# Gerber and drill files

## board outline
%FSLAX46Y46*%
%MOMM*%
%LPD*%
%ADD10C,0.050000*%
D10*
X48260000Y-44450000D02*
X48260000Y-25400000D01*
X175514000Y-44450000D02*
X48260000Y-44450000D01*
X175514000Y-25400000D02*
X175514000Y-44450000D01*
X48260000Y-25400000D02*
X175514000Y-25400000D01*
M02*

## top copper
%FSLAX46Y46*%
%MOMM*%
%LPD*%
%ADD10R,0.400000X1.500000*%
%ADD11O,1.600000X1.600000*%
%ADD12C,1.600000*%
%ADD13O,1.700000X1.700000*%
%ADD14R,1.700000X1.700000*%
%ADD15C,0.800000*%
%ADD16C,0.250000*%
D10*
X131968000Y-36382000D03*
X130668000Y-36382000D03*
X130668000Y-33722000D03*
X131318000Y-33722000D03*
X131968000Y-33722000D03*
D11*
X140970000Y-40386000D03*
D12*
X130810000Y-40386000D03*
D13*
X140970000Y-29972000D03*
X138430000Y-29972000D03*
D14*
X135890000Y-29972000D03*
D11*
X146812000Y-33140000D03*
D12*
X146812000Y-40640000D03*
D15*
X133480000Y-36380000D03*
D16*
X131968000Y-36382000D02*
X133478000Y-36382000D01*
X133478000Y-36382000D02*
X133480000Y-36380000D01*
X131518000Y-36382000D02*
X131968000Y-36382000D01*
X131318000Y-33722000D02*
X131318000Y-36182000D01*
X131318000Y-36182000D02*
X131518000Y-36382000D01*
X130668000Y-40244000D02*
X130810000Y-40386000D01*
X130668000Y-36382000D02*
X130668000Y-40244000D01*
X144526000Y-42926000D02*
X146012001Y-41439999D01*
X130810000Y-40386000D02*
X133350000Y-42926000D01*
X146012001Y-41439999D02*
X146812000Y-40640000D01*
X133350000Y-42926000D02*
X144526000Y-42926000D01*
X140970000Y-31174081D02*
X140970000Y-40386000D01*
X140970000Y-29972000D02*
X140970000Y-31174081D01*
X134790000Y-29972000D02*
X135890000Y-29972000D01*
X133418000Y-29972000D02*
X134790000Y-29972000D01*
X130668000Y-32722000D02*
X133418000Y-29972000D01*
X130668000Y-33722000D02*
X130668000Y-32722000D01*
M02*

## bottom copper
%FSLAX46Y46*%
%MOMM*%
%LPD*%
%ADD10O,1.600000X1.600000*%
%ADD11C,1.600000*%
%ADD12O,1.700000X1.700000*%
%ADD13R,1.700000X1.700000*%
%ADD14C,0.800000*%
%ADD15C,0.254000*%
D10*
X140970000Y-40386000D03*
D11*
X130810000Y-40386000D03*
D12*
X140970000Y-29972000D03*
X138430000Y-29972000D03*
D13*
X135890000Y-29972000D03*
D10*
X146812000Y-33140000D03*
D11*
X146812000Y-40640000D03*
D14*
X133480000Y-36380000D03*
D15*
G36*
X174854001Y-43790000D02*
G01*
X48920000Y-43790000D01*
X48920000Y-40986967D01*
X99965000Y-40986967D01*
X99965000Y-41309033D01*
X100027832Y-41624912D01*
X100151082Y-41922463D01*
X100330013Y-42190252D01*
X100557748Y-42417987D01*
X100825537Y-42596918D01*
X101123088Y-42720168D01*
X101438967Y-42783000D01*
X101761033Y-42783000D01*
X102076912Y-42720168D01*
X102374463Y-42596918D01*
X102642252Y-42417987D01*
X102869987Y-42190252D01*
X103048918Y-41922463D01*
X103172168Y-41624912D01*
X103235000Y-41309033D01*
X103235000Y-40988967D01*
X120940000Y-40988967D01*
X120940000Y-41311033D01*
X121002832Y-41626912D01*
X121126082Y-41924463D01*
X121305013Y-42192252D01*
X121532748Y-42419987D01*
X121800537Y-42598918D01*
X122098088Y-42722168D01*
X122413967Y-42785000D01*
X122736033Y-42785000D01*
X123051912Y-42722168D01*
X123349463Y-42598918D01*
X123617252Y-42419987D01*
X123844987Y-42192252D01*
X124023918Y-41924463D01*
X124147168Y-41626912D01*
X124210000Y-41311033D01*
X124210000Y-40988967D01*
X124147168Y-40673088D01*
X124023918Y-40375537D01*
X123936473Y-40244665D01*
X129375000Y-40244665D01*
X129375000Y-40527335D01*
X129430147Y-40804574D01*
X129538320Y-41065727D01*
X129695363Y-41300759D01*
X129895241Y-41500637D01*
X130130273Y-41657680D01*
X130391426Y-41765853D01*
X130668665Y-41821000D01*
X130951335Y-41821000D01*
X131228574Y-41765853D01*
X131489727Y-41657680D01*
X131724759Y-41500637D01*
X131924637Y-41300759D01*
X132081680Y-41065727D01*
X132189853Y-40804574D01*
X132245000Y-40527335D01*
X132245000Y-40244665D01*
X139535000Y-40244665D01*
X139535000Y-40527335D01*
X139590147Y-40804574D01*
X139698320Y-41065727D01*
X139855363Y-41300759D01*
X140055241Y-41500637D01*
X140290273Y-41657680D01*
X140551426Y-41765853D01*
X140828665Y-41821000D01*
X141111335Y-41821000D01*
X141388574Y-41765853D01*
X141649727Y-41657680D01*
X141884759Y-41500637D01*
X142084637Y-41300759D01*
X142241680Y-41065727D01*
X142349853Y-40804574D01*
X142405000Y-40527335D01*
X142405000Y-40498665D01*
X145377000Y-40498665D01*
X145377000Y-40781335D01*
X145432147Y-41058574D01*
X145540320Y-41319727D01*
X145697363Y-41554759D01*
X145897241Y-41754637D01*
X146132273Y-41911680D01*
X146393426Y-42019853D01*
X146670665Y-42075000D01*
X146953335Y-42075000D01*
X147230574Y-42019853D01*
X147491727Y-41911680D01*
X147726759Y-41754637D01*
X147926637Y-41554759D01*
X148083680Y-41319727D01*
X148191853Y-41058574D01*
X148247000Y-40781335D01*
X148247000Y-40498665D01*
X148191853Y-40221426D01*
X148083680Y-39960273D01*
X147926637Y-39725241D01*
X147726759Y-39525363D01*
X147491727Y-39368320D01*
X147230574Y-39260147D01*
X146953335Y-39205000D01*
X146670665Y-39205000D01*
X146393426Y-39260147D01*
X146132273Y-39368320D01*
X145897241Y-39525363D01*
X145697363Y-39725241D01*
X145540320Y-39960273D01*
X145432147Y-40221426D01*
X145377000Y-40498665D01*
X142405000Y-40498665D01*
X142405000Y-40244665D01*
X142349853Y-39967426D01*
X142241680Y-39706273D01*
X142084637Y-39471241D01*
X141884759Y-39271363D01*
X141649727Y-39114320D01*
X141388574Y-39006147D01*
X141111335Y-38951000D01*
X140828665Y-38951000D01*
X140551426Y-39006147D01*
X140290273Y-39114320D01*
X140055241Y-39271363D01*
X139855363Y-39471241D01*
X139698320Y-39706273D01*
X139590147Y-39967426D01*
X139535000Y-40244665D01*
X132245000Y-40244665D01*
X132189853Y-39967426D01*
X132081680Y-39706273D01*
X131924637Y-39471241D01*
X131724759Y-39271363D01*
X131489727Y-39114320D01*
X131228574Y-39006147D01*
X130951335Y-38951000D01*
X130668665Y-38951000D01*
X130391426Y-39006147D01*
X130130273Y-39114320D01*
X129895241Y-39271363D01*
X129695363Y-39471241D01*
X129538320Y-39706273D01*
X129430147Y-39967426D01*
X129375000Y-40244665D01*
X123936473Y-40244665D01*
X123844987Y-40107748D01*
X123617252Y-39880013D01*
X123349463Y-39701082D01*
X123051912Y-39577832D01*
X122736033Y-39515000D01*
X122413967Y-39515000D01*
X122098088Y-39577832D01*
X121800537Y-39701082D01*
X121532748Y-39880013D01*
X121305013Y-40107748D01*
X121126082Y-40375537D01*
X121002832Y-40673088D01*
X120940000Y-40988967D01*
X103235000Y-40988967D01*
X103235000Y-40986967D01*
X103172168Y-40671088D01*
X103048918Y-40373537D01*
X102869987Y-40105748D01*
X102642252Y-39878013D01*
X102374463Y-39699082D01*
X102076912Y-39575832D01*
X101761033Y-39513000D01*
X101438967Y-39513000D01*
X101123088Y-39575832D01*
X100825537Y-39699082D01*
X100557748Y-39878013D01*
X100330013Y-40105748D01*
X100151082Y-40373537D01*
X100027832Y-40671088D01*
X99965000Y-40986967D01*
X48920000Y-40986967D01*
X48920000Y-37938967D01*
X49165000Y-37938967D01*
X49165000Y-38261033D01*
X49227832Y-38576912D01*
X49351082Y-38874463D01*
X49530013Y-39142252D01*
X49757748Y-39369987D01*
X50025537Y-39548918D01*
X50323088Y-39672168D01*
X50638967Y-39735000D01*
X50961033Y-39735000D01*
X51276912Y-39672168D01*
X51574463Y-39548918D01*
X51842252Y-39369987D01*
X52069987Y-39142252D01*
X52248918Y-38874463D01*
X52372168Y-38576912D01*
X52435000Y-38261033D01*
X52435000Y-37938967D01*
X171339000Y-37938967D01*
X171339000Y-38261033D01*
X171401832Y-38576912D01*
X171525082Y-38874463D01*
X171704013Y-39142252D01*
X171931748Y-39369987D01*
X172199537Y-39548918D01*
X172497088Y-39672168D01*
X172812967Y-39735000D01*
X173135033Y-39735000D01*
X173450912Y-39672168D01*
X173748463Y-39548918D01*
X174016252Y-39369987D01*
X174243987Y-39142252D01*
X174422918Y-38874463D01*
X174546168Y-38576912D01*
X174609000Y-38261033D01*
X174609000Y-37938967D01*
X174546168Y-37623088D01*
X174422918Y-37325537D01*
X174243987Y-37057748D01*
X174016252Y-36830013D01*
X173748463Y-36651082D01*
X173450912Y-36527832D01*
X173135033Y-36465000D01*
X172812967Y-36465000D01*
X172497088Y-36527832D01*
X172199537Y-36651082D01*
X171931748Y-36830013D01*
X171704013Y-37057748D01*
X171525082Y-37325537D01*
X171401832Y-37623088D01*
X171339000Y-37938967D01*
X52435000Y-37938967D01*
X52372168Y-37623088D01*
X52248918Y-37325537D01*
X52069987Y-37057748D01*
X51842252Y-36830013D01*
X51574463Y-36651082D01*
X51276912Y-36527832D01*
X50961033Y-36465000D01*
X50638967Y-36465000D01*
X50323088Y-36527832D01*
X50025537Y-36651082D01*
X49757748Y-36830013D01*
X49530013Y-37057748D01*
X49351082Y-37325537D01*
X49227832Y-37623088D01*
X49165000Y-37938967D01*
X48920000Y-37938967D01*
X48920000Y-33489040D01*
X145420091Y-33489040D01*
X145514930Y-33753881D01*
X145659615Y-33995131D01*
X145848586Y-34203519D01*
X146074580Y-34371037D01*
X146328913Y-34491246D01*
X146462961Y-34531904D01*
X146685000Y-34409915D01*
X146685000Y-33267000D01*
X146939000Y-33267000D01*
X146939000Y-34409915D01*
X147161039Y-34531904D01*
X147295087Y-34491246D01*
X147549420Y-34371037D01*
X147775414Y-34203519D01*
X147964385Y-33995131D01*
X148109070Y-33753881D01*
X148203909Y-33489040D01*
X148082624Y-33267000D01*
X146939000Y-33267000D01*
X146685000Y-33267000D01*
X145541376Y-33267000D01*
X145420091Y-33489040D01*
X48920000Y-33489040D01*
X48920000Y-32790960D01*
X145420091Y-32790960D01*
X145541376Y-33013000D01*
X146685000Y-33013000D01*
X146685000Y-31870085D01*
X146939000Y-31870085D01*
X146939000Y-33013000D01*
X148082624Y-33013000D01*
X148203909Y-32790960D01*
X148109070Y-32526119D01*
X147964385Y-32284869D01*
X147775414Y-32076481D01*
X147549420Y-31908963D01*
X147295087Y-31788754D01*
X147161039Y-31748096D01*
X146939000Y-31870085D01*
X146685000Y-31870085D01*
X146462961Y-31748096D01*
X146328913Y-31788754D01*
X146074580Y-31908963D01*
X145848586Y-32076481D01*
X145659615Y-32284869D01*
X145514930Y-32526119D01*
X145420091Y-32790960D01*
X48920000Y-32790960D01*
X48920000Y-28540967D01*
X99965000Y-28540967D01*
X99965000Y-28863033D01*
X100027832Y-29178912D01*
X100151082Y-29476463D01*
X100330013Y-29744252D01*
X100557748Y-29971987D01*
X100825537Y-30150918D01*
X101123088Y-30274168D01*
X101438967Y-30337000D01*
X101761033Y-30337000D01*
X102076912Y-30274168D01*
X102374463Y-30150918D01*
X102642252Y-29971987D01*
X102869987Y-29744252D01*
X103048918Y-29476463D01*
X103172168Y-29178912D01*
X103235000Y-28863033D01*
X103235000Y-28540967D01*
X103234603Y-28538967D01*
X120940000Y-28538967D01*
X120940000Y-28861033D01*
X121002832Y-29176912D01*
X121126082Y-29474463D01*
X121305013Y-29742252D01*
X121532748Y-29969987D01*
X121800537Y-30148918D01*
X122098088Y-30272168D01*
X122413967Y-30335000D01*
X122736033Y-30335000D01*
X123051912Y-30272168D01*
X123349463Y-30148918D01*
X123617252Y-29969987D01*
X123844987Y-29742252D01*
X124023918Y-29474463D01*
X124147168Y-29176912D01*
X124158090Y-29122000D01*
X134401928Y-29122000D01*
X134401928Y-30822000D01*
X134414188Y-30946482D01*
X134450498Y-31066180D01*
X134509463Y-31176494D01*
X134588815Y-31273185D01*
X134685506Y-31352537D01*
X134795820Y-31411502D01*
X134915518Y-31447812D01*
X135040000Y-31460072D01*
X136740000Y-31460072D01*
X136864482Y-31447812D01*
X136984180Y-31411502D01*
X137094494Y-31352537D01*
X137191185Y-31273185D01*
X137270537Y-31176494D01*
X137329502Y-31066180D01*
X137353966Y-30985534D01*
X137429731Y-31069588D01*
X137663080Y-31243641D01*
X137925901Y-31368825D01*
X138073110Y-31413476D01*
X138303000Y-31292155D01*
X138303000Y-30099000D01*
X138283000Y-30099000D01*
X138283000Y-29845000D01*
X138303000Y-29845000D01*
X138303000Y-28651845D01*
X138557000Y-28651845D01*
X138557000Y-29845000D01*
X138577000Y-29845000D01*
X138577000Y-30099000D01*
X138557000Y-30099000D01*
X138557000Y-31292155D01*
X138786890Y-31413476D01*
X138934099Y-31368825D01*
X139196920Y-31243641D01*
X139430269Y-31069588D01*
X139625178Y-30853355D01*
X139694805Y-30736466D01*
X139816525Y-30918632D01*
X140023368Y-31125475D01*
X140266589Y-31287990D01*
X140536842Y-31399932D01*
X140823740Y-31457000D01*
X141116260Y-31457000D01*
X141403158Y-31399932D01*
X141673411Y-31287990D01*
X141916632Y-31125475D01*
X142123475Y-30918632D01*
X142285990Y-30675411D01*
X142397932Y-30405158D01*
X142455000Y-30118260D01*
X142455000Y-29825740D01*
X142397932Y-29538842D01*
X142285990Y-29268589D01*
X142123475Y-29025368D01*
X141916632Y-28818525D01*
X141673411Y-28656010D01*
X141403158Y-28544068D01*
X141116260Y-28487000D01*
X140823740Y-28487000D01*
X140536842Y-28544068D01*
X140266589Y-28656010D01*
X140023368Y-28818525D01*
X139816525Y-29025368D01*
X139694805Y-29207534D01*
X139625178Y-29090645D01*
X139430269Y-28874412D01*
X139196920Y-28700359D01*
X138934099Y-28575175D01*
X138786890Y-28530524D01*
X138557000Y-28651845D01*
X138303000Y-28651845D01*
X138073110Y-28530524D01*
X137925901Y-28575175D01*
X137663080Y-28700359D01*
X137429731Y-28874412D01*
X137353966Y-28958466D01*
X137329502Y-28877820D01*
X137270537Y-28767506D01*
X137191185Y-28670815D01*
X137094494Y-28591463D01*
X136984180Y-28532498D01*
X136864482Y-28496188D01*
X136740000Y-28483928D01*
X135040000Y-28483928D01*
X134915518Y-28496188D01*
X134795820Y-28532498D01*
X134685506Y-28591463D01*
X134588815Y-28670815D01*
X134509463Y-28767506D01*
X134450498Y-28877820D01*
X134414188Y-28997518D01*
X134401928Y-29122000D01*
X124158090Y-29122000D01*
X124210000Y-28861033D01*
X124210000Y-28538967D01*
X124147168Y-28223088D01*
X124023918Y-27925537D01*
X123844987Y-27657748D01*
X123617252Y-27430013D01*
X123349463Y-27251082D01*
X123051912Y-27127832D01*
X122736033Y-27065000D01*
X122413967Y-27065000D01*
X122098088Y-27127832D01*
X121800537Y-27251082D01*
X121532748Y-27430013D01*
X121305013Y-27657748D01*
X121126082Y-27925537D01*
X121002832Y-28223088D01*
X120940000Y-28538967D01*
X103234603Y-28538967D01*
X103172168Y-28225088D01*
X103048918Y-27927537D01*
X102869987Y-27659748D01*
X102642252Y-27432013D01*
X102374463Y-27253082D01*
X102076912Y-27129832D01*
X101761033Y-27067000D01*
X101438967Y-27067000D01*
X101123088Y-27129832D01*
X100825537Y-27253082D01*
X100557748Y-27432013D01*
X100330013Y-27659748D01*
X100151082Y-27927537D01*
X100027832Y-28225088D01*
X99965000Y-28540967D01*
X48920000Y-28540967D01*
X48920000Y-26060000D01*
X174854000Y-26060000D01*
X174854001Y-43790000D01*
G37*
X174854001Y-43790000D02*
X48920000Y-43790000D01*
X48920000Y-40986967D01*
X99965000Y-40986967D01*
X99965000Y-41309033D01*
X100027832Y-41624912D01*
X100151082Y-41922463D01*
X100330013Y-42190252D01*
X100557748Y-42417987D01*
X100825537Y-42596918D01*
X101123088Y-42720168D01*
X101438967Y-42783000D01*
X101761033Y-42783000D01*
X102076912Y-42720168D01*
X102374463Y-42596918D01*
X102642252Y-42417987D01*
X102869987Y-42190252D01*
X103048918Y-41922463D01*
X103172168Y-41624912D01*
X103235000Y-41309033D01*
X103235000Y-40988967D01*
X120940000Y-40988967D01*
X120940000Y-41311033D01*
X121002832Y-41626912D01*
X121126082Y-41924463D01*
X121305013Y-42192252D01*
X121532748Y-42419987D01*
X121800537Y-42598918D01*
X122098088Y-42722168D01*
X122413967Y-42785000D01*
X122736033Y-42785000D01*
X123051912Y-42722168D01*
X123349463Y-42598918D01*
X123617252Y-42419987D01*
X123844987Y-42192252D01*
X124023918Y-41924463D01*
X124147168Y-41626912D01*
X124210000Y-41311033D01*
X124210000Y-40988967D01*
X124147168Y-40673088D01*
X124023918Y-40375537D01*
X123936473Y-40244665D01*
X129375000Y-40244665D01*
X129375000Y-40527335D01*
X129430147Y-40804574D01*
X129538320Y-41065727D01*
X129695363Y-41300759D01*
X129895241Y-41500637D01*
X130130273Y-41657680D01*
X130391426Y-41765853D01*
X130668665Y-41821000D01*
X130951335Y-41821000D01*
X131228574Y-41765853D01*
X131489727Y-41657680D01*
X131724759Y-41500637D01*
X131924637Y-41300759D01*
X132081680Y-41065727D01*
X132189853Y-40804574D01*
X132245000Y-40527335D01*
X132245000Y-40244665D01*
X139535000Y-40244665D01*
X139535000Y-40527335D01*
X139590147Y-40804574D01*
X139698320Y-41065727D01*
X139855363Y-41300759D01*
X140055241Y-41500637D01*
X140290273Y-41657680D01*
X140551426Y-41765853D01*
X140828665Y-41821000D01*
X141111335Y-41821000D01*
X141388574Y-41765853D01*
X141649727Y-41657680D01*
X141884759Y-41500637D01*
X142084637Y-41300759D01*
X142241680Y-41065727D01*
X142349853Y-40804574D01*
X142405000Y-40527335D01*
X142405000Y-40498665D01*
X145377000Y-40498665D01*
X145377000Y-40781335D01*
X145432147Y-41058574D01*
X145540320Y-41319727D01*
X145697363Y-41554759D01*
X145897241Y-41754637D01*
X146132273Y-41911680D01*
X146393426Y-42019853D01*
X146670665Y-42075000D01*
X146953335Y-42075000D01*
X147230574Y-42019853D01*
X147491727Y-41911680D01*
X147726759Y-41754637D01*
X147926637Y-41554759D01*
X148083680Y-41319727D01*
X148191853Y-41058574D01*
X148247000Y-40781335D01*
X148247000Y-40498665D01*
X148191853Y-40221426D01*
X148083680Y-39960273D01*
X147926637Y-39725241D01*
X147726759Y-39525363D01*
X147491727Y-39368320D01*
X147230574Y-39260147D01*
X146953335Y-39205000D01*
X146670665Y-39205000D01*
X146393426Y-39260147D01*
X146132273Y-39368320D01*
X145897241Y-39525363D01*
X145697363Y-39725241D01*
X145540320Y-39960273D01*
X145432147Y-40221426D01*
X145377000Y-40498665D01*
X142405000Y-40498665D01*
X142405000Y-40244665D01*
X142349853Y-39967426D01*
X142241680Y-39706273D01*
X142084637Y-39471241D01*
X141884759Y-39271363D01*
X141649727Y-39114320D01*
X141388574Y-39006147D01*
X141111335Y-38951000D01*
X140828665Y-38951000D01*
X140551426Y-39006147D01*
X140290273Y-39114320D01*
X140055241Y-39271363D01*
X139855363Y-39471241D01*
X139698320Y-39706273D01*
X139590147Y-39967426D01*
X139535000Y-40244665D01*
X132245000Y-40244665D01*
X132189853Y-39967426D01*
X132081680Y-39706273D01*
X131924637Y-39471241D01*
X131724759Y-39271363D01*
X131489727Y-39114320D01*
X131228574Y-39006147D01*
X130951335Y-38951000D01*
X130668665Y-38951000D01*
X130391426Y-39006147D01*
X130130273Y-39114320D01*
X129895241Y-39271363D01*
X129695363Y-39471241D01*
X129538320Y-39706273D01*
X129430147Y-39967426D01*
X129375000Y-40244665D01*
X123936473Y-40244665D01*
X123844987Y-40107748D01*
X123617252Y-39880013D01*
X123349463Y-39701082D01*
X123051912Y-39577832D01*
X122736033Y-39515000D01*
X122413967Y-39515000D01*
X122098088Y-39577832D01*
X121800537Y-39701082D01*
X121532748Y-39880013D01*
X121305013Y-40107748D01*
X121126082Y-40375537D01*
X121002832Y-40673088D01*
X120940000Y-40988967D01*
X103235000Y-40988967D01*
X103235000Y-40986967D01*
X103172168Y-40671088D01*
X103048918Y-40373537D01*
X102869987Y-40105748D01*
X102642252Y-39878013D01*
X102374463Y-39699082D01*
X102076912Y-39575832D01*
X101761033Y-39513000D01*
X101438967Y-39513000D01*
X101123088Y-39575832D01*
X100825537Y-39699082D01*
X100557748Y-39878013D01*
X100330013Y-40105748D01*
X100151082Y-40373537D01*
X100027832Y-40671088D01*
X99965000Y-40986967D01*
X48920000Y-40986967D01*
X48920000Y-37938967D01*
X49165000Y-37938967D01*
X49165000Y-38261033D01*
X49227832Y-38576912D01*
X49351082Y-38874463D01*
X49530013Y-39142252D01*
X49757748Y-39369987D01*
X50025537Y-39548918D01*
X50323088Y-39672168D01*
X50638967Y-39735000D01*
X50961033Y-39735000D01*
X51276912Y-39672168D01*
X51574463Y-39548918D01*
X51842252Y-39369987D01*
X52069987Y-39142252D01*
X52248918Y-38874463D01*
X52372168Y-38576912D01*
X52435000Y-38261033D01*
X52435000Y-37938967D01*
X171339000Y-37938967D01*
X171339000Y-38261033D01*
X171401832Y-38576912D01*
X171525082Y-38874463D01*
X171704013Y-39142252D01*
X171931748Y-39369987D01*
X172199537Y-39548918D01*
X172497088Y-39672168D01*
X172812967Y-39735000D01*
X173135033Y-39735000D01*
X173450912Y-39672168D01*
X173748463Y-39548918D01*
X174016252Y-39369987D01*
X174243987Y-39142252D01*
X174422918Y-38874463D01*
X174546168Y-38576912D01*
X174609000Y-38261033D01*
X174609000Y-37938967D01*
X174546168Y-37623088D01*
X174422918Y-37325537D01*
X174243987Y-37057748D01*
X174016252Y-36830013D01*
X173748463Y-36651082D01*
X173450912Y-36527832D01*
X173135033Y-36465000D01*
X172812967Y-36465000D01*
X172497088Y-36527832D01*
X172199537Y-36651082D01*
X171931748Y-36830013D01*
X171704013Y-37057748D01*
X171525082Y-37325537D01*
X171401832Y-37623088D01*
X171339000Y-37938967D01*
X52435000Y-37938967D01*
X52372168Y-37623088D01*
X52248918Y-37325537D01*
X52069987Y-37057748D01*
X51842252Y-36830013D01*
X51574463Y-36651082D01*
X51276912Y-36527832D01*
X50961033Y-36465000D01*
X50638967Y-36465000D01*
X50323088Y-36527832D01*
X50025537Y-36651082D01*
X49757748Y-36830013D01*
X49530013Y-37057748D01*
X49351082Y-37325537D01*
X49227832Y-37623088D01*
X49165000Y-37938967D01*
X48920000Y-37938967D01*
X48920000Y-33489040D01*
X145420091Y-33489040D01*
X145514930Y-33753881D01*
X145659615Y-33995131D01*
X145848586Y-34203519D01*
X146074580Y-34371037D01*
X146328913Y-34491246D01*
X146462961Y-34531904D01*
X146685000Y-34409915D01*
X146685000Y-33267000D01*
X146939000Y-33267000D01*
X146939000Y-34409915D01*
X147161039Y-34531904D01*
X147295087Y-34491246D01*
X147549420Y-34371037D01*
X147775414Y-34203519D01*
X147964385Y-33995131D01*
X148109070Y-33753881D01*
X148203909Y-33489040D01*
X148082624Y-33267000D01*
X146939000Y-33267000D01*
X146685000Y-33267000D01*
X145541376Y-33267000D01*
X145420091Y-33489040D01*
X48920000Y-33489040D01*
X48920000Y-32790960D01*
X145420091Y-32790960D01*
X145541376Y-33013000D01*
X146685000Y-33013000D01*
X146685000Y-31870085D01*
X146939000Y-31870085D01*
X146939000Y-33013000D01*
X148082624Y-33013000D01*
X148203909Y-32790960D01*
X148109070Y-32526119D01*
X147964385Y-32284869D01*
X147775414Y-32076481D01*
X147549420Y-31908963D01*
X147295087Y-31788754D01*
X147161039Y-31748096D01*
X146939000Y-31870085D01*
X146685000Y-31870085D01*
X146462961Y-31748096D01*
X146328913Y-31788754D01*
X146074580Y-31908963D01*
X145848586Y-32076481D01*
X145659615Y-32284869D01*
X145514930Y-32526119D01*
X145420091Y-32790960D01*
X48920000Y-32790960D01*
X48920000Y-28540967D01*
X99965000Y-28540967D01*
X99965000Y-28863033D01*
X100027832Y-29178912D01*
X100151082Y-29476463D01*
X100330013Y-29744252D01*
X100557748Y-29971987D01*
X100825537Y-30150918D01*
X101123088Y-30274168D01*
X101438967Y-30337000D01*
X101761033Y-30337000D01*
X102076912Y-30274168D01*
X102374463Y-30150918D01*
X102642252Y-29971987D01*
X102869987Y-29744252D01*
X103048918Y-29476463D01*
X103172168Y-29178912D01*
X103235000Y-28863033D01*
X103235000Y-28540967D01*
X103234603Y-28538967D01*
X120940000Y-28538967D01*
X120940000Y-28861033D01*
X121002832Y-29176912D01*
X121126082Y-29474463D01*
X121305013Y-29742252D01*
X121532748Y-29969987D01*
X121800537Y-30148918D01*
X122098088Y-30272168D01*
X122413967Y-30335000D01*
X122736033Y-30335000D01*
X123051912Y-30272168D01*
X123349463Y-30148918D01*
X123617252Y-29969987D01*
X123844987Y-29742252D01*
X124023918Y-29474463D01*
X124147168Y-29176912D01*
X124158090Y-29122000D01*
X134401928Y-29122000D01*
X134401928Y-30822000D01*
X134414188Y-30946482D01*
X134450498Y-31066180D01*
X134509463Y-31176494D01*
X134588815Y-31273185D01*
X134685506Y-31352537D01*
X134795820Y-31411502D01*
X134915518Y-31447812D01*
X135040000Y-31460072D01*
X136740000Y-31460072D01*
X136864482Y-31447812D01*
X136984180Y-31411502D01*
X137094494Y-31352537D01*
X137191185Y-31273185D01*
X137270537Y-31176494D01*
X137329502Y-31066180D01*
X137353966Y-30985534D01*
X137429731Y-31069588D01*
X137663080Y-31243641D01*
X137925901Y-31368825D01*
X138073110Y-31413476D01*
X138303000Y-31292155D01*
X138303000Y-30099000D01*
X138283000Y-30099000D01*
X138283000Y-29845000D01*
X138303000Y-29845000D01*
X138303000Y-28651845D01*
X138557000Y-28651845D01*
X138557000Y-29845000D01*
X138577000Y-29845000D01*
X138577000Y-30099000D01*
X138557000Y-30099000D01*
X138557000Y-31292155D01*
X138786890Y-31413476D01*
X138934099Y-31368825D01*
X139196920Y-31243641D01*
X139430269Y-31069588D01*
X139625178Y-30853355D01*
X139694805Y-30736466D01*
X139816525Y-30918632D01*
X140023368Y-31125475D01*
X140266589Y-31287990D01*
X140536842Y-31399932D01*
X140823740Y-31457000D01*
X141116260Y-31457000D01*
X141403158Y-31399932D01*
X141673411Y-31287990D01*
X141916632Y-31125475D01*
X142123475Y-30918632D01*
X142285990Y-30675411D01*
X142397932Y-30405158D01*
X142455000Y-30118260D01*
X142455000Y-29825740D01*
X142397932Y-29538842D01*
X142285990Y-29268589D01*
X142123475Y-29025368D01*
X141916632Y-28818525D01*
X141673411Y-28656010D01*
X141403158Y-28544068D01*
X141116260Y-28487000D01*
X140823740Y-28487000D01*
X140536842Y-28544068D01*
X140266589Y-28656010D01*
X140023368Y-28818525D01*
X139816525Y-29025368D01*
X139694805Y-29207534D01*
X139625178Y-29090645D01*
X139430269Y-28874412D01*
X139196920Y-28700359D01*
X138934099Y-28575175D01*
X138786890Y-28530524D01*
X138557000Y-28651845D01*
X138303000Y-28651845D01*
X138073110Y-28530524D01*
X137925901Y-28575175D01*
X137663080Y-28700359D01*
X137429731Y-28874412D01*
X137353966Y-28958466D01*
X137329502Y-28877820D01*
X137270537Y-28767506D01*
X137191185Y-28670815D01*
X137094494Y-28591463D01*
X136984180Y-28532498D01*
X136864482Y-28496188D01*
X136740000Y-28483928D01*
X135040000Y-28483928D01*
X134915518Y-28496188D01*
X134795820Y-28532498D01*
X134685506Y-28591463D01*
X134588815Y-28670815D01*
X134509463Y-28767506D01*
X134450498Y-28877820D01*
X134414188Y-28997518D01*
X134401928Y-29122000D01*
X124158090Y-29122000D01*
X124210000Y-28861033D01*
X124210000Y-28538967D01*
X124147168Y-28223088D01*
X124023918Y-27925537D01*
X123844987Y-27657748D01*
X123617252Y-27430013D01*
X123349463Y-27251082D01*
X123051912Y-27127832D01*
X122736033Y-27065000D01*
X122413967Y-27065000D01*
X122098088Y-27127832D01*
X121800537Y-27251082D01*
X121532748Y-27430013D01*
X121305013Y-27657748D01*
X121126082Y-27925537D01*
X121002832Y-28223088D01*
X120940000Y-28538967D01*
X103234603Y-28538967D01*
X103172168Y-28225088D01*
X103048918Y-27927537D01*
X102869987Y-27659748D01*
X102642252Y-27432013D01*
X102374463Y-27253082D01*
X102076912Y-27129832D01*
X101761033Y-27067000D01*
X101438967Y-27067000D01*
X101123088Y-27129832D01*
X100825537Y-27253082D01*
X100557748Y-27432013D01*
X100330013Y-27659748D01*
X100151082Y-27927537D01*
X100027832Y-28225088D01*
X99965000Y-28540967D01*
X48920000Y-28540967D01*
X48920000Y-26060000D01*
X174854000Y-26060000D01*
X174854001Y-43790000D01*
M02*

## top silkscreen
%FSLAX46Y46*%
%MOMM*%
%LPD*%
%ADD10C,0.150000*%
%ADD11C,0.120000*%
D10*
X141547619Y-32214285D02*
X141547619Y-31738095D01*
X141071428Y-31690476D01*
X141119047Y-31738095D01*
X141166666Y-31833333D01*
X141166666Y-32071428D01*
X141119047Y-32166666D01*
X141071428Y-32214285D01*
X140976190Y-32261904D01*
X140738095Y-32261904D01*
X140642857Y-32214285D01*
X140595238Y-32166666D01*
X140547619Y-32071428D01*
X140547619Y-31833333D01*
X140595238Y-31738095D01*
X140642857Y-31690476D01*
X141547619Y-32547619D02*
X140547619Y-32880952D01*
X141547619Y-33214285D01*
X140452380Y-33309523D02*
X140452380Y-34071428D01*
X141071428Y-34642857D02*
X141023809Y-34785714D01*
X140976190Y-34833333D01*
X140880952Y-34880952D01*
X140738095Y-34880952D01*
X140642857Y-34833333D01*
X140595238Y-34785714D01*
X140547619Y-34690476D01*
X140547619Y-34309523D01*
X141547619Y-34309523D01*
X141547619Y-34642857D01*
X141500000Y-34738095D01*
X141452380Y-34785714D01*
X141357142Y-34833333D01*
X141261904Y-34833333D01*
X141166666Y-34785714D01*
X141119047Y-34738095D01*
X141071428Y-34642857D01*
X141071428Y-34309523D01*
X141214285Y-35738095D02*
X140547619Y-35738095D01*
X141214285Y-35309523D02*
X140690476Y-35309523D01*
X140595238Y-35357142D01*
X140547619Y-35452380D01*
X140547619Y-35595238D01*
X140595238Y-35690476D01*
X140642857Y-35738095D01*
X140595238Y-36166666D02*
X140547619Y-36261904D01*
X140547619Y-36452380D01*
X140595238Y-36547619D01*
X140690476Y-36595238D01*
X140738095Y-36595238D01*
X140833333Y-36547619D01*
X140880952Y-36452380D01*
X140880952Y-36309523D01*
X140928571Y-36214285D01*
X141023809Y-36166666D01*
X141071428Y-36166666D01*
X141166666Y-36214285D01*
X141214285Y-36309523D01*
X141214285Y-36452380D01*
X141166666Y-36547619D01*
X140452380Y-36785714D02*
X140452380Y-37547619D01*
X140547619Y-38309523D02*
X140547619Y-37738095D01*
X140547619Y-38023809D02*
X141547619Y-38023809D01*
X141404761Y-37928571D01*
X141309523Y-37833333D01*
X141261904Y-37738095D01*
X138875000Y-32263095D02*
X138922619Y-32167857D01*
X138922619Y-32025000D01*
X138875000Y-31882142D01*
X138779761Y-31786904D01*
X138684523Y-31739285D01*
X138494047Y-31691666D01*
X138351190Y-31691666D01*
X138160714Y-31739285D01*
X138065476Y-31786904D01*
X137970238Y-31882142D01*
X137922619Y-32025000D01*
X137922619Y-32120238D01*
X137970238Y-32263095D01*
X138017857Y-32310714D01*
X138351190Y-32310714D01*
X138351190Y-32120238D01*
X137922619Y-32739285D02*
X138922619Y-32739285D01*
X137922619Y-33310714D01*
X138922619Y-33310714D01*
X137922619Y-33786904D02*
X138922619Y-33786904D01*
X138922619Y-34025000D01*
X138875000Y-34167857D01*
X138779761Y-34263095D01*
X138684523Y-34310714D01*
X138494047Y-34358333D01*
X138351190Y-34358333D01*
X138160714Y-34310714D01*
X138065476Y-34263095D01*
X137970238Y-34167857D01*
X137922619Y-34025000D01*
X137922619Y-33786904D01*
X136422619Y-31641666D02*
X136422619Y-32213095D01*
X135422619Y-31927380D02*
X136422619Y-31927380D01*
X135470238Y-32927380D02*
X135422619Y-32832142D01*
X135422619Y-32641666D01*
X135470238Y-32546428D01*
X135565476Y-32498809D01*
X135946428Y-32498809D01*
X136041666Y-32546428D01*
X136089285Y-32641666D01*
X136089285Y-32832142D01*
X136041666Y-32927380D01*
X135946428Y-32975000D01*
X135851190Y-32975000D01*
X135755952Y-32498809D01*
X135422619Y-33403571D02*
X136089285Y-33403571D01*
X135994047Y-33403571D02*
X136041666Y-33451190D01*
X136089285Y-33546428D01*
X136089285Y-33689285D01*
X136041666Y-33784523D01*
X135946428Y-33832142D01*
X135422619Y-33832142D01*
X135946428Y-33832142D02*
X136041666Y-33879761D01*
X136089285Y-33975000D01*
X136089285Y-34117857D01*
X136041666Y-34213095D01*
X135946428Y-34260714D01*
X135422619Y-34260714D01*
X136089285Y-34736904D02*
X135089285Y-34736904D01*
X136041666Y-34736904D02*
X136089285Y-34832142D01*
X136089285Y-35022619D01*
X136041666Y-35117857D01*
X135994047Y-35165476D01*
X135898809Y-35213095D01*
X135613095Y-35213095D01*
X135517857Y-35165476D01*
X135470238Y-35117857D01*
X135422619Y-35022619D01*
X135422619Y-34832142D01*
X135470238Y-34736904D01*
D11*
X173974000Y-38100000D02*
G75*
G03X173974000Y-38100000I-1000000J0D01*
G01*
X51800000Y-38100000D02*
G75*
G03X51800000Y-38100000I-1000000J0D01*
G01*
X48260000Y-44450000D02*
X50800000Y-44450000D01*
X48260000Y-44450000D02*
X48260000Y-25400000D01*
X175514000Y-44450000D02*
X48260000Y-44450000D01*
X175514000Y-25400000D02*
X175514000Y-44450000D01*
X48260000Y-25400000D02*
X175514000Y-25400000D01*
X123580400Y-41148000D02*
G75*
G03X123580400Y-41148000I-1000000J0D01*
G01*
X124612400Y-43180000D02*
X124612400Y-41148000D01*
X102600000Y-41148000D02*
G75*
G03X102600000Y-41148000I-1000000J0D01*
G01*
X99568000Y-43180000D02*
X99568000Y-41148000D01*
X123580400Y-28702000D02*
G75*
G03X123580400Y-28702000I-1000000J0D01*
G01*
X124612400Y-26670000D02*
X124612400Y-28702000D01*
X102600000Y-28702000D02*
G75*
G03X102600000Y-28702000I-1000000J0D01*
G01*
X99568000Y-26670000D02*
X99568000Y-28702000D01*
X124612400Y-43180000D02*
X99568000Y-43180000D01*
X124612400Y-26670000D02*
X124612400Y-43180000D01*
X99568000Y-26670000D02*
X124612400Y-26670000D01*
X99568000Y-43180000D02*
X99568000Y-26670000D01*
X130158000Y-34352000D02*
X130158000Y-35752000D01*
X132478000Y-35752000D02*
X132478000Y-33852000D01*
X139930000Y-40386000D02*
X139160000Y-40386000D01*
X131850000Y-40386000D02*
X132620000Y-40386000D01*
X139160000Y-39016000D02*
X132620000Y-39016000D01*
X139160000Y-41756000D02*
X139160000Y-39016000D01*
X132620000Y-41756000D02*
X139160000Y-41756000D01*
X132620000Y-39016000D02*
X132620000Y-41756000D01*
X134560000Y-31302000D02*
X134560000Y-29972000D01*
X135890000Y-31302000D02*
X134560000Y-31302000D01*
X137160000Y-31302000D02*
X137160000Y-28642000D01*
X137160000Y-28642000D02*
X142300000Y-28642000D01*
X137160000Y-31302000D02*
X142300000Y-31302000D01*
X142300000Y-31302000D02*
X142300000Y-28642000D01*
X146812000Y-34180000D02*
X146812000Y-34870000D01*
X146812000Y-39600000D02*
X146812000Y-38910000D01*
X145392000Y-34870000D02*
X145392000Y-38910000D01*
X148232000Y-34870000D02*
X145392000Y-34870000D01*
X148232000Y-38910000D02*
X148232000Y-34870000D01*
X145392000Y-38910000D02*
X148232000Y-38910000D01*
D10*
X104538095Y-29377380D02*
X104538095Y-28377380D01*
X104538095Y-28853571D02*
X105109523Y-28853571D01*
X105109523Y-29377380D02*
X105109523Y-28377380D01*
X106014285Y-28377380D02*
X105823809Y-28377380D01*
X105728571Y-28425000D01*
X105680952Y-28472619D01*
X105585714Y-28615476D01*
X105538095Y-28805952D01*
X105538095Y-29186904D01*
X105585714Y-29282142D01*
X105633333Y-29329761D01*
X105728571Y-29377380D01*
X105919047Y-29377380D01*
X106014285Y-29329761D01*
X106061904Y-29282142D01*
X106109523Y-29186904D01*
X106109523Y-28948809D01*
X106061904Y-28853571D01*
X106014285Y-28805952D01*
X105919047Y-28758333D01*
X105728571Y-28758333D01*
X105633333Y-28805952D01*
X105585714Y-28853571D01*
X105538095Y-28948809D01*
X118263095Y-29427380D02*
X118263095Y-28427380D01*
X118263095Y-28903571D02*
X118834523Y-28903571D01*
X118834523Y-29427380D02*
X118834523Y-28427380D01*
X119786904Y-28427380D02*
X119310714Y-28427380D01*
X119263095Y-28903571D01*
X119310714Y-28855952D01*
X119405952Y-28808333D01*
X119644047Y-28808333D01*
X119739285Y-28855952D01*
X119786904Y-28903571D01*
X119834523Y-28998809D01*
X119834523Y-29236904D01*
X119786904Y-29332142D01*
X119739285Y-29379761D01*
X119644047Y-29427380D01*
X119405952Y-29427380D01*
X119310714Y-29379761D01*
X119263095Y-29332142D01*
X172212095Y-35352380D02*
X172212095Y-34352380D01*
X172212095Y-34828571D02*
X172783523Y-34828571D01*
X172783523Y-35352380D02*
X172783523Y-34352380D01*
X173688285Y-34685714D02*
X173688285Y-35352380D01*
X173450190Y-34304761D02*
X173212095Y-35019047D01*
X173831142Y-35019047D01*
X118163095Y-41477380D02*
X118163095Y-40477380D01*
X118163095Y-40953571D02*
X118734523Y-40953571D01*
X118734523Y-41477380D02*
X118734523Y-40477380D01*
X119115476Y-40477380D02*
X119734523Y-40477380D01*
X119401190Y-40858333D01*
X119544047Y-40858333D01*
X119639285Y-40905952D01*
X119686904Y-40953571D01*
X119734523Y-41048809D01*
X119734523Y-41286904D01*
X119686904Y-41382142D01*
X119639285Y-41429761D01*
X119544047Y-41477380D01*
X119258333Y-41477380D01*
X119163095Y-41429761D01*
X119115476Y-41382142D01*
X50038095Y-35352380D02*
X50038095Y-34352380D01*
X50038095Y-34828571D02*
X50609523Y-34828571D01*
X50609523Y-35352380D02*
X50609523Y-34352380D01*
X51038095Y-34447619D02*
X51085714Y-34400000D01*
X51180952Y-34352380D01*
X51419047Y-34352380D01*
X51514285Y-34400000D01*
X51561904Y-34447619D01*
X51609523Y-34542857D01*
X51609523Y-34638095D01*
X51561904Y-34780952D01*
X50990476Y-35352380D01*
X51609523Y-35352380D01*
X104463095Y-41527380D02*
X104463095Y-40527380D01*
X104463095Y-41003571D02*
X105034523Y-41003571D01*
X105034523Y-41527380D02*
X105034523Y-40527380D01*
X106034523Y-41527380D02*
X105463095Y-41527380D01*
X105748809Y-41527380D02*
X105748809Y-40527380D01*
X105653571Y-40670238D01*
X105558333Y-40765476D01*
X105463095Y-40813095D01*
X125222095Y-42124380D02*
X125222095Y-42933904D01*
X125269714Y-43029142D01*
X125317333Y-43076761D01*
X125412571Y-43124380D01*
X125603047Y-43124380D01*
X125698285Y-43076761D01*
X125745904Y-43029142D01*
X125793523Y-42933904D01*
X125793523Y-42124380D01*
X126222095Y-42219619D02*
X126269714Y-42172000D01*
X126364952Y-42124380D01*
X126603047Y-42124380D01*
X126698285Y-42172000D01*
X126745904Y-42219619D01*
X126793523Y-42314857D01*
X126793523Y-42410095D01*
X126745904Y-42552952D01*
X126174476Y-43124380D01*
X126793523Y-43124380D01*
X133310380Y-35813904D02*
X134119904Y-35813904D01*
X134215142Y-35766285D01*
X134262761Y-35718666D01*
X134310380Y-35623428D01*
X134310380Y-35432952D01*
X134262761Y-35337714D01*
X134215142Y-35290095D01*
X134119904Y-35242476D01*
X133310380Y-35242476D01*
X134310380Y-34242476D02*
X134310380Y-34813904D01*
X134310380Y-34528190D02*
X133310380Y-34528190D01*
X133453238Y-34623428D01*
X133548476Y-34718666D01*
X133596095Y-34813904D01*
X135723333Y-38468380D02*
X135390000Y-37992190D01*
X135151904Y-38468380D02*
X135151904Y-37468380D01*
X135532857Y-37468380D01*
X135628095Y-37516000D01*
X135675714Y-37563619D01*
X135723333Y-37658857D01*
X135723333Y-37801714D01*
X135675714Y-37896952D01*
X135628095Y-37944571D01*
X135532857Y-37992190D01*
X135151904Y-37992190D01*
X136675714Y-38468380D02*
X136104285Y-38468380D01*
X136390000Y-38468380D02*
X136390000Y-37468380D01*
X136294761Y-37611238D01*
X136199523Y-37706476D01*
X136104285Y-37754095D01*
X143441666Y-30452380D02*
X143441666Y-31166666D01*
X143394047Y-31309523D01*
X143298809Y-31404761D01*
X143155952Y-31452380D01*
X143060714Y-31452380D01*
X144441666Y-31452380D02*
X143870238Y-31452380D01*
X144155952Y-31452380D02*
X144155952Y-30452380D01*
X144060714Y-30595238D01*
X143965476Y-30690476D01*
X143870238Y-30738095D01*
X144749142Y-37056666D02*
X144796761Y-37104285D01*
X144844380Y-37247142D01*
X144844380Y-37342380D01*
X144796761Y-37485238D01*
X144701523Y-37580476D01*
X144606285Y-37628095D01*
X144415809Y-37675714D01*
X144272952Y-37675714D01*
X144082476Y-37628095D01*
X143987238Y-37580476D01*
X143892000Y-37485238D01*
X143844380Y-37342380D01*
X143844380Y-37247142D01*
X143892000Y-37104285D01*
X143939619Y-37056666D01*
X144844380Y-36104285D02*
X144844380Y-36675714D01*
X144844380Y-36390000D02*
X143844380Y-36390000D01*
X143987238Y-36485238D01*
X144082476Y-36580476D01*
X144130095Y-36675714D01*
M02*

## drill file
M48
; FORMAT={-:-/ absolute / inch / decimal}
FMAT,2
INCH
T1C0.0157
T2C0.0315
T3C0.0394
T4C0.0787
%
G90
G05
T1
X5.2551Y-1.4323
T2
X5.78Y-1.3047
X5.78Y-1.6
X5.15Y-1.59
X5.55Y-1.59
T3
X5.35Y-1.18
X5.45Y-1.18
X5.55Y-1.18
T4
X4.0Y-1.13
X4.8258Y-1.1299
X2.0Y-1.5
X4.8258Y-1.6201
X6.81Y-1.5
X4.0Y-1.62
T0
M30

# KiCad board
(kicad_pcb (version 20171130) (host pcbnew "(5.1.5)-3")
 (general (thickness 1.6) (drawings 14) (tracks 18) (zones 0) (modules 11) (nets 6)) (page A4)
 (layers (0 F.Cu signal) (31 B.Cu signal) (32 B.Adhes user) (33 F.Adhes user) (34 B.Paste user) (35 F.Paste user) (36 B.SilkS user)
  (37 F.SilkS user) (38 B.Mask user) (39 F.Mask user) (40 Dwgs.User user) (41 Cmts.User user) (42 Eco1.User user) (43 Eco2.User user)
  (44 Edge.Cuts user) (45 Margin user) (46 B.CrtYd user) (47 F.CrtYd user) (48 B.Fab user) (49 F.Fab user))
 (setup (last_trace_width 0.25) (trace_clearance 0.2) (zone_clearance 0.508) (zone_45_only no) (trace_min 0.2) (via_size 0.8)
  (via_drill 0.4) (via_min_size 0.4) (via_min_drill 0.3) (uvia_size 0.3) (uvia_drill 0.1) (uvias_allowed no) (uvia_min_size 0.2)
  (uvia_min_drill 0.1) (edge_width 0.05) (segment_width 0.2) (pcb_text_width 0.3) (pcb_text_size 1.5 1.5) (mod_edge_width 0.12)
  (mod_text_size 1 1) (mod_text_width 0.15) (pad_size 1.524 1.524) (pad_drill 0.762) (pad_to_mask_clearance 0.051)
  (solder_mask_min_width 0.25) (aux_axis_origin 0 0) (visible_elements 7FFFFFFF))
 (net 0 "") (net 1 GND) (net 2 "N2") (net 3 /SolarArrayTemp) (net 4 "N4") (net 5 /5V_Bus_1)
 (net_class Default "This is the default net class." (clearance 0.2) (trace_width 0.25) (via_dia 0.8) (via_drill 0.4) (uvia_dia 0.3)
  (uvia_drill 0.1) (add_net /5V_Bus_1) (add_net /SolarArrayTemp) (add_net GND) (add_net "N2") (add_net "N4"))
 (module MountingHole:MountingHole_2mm (layer F.Cu) (at 101.6 28.702)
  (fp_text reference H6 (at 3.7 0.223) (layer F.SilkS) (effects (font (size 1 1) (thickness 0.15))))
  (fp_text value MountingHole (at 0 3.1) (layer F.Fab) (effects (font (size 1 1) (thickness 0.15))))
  (pad "" np_thru_hole circle (at 0 0) (size 2 2) (drill 2) (layers *.Cu *.Mask)))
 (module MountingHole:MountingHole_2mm (layer F.Cu) (at 122.575 28.7)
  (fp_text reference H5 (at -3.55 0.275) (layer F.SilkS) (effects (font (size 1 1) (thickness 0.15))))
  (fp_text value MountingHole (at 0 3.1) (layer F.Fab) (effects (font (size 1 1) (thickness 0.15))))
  (pad "" np_thru_hole circle (at 0 0) (size 2 2) (drill 2) (layers *.Cu *.Mask)))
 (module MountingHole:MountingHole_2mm (layer F.Cu) (at 172.974 38.1)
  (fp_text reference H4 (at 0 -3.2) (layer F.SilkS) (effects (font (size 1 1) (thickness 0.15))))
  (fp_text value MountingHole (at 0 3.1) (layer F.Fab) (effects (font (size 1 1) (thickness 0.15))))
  (pad "" np_thru_hole circle (at 0 0) (size 2 2) (drill 2) (layers *.Cu *.Mask)))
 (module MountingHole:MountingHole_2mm (layer F.Cu) (at 122.575 41.15)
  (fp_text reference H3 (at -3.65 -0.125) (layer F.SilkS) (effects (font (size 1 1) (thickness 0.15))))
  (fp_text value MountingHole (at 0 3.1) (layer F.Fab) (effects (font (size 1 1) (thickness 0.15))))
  (pad "" np_thru_hole circle (at 0 0) (size 2 2) (drill 2) (layers *.Cu *.Mask)))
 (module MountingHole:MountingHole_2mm (layer F.Cu) (at 50.8 38.1)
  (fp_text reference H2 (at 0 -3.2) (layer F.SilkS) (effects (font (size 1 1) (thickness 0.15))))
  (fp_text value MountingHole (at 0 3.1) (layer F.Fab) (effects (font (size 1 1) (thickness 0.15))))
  (pad "" np_thru_hole circle (at 0 0) (size 2 2) (drill 2) (layers *.Cu *.Mask)))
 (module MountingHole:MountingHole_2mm (layer F.Cu) (at 101.6 41.148)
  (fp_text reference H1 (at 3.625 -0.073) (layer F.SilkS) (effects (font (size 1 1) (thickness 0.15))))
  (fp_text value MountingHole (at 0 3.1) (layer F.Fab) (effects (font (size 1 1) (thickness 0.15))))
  (pad "" np_thru_hole circle (at 0 0) (size 2 2) (drill 2) (layers *.Cu *.Mask)))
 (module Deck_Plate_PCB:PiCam (layer F.Cu) (at 99.568 43.18)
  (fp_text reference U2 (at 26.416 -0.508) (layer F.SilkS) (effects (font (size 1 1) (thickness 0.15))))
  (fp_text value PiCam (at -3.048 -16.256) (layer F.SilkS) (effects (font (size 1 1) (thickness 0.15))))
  (fp_circle (center 23.0124 -2.032) (end 24.0124 -2.032) (layer F.SilkS) (width 0.12))
  (fp_line (start 25.0444 0) (end 25.0444 -2.032) (layer F.SilkS) (width 0.12))
  (fp_circle (center 2.032 -2.032) (end 3.032 -2.032) (layer F.SilkS) (width 0.12))
  (fp_line (start 0 0) (end 0 -2.032) (layer F.SilkS) (width 0.12))
  (fp_circle (center 23.0124 -14.478) (end 24.0124 -14.478) (layer F.SilkS) (width 0.12))
  (fp_line (start 25.0444 -16.51) (end 25.0444 -14.478) (layer F.SilkS) (width 0.12))
  (fp_circle (center 2.032 -14.478) (end 3.032 -14.478) (layer F.SilkS) (width 0.12))
  (fp_line (start 0 -16.51) (end 0 -14.478) (layer F.SilkS) (width 0.12))
  (fp_line (start 25.0444 0) (end 0 0) (layer F.SilkS) (width 0.12))
  (fp_line (start 25.0444 -16.51) (end 25.0444 0) (layer F.SilkS) (width 0.12))
  (fp_line (start 0 -16.51) (end 25.0444 -16.51) (layer F.SilkS) (width 0.12))
  (fp_line (start 0 0) (end 0 -16.51) (layer F.SilkS) (width 0.12)))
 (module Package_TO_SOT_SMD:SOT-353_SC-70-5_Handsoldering (layer F.Cu) (at 131.318 35.052 270)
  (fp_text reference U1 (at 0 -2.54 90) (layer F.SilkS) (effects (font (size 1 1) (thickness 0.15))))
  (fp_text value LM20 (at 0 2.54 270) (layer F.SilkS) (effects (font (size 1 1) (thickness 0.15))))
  (fp_line (start -0.7 1.16) (end 0.7 1.16) (layer F.SilkS) (width 0.12))
  (fp_line (start 0.7 -1.16) (end -1.2 -1.16) (layer F.SilkS) (width 0.12))
  (pad 5 smd rect (at 1.33 -0.65 270) (size 1.5 0.4) (layers F.Cu F.Paste F.Mask) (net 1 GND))
  (pad 4 smd rect (at 1.33 0.65 270) (size 1.5 0.4) (layers F.Cu F.Paste F.Mask) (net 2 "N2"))
  (pad 3 smd rect (at -1.33 0.65 270) (size 1.5 0.4) (layers F.Cu F.Paste F.Mask) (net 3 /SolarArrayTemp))
  (pad 2 smd rect (at -1.33 0 270) (size 1.5 0.4) (layers F.Cu F.Paste F.Mask) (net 1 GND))
  (pad 1 smd rect (at -1.33 -0.65 270) (size 1.5 0.4) (layers F.Cu F.Paste F.Mask) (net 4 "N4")))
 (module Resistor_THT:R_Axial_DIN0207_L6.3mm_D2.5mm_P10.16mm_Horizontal (layer F.Cu) (at 130.81 40.386)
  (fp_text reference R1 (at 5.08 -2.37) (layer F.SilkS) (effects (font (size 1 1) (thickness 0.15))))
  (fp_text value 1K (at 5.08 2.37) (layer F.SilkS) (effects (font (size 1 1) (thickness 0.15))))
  (fp_line (start 9.12 0) (end 8.35 0) (layer F.SilkS) (width 0.12))
  (fp_line (start 1.04 0) (end 1.81 0) (layer F.SilkS) (width 0.12))
  (fp_line (start 8.35 -1.37) (end 1.81 -1.37) (layer F.SilkS) (width 0.12))
  (fp_line (start 8.35 1.37) (end 8.35 -1.37) (layer F.SilkS) (width 0.12))
  (fp_line (start 1.81 1.37) (end 8.35 1.37) (layer F.SilkS) (width 0.12))
  (fp_line (start 1.81 -1.37) (end 1.81 1.37) (layer F.SilkS) (width 0.12))
  (pad 2 thru_hole oval (at 10.16 0) (size 1.6 1.6) (drill 0.8) (layers *.Cu *.Mask) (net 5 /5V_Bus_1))
  (pad 1 thru_hole circle (at 0 0) (size 1.6 1.6) (drill 0.8) (layers *.Cu *.Mask) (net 2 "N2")))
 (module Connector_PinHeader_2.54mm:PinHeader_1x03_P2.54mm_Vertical (layer F.Cu) (at 135.89 29.972 90)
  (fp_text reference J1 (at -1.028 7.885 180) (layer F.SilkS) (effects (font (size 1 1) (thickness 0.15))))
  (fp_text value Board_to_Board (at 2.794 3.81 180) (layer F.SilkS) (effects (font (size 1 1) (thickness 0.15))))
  (fp_line (start -1.33 -1.33) (end 0 -1.33) (layer F.SilkS) (width 0.12))
  (fp_line (start -1.33 0) (end -1.33 -1.33) (layer F.SilkS) (width 0.12))
  (fp_line (start -1.33 1.27) (end 1.33 1.27) (layer F.SilkS) (width 0.12))
  (fp_line (start 1.33 1.27) (end 1.33 6.41) (layer F.SilkS) (width 0.12))
  (fp_line (start -1.33 1.27) (end -1.33 6.41) (layer F.SilkS) (width 0.12))
  (fp_line (start -1.33 6.41) (end 1.33 6.41) (layer F.SilkS) (width 0.12))
  (pad 3 thru_hole oval (at 0 5.08 90) (size 1.7 1.7) (drill 1) (layers *.Cu *.Mask) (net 5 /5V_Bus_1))
  (pad 2 thru_hole oval (at 0 2.54 90) (size 1.7 1.7) (drill 1) (layers *.Cu *.Mask) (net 1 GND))
  (pad 1 thru_hole rect (at 0 0 90) (size 1.7 1.7) (drill 1) (layers *.Cu *.Mask) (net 3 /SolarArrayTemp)))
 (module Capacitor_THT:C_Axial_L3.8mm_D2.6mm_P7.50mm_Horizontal (layer F.Cu) (at 146.812 40.64 90)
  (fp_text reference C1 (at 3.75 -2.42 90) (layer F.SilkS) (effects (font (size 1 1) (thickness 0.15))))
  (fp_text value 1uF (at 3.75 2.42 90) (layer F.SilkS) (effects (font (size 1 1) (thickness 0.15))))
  (fp_line (start 6.46 0) (end 5.77 0) (layer F.SilkS) (width 0.12))
  (fp_line (start 1.04 0) (end 1.73 0) (layer F.SilkS) (width 0.12))
  (fp_line (start 5.77 -1.42) (end 1.73 -1.42) (layer F.SilkS) (width 0.12))
  (fp_line (start 5.77 1.42) (end 5.77 -1.42) (layer F.SilkS) (width 0.12))
  (fp_line (start 1.73 1.42) (end 5.77 1.42) (layer F.SilkS) (width 0.12))
  (fp_line (start 1.73 -1.42) (end 1.73 1.42) (layer F.SilkS) (width 0.12))
  (pad 2 thru_hole oval (at 7.5 0 90) (size 1.6 1.6) (drill 0.8) (layers *.Cu *.Mask) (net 1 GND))
  (pad 1 thru_hole circle (at 0 0 90) (size 1.6 1.6) (drill 0.8) (layers *.Cu *.Mask) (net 2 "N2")))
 (gr_line (start 48.26 44.45) (end 48.26 25.4) (layer Edge.Cuts) (width 0.05))
 (gr_line (start 175.514 44.45) (end 48.26 44.45) (layer Edge.Cuts) (width 0.05))
 (gr_line (start 175.514 25.4) (end 175.514 44.45) (layer Edge.Cuts) (width 0.05))
 (gr_line (start 48.26 25.4) (end 175.514 25.4) (layer Edge.Cuts) (width 0.05))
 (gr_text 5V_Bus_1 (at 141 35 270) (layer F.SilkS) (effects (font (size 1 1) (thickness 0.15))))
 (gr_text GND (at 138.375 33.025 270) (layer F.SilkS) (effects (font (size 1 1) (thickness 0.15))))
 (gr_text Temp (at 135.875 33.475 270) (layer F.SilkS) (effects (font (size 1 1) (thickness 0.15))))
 (gr_circle (center 172.974 38.1) (end 173.974 38.1) (layer F.SilkS) (width 0.12))
 (gr_circle (center 50.8 38.1) (end 51.8 38.1) (layer F.SilkS) (width 0.12))
 (gr_line (start 48.26 44.45) (end 50.8 44.45) (layer F.SilkS) (width 0.12))
 (gr_line (start 48.26 44.45) (end 48.26 25.4) (layer F.SilkS) (width 0.12))
 (gr_line (start 175.514 44.45) (end 48.26 44.45) (layer F.SilkS) (width 0.12))
 (gr_line (start 175.514 25.4) (end 175.514 44.45) (layer F.SilkS) (width 0.12))
 (gr_line (start 48.26 25.4) (end 175.514 25.4) (layer F.SilkS) (width 0.12))
 (via (at 133.48 36.38) (size 0.8) (drill 0.4) (layers F.Cu B.Cu) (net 1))
 (segment (start 131.968 36.382) (end 133.478 36.382) (width 0.25) (layer F.Cu) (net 1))
 (segment (start 133.478 36.382) (end 133.48 36.38) (width 0.25) (layer F.Cu) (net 1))
 (segment (start 131.518 36.382) (end 131.968 36.382) (width 0.25) (layer F.Cu) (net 1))
 (segment (start 131.318 33.722) (end 131.318 36.182) (width 0.25) (layer F.Cu) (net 1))
 (segment (start 131.318 36.182) (end 131.518 36.382) (width 0.25) (layer F.Cu) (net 1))
 (segment (start 130.668 40.244) (end 130.81 40.386) (width 0.25) (layer F.Cu) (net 2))
 (segment (start 130.668 36.382) (end 130.668 40.244) (width 0.25) (layer F.Cu) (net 2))
 (segment (start 144.526 42.926) (end 146.012001 41.439999) (width 0.25) (layer F.Cu) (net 2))
 (segment (start 130.81 40.386) (end 133.35 42.926) (width 0.25) (layer F.Cu) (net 2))
 (segment (start 146.012001 41.439999) (end 146.812 40.64) (width 0.25) (layer F.Cu) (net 2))
 (segment (start 133.35 42.926) (end 144.526 42.926) (width 0.25) (layer F.Cu) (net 2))
 (segment (start 140.97 31.174081) (end 140.97 40.386) (width 0.25) (layer F.Cu) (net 5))
 (segment (start 140.97 29.972) (end 140.97 31.174081) (width 0.25) (layer F.Cu) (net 5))
 (segment (start 134.79 29.972) (end 135.89 29.972) (width 0.25) (layer F.Cu) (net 3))
 (segment (start 133.418 29.972) (end 134.79 29.972) (width 0.25) (layer F.Cu) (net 3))
 (segment (start 130.668 32.722) (end 133.418 29.972) (width 0.25) (layer F.Cu) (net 3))
 (segment (start 130.668 33.722) (end 130.668 32.722) (width 0.25) (layer F.Cu) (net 3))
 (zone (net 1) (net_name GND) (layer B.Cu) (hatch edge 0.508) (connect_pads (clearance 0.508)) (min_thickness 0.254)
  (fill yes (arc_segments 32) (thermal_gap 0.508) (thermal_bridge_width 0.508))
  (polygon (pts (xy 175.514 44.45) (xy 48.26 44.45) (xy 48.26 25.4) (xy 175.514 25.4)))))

